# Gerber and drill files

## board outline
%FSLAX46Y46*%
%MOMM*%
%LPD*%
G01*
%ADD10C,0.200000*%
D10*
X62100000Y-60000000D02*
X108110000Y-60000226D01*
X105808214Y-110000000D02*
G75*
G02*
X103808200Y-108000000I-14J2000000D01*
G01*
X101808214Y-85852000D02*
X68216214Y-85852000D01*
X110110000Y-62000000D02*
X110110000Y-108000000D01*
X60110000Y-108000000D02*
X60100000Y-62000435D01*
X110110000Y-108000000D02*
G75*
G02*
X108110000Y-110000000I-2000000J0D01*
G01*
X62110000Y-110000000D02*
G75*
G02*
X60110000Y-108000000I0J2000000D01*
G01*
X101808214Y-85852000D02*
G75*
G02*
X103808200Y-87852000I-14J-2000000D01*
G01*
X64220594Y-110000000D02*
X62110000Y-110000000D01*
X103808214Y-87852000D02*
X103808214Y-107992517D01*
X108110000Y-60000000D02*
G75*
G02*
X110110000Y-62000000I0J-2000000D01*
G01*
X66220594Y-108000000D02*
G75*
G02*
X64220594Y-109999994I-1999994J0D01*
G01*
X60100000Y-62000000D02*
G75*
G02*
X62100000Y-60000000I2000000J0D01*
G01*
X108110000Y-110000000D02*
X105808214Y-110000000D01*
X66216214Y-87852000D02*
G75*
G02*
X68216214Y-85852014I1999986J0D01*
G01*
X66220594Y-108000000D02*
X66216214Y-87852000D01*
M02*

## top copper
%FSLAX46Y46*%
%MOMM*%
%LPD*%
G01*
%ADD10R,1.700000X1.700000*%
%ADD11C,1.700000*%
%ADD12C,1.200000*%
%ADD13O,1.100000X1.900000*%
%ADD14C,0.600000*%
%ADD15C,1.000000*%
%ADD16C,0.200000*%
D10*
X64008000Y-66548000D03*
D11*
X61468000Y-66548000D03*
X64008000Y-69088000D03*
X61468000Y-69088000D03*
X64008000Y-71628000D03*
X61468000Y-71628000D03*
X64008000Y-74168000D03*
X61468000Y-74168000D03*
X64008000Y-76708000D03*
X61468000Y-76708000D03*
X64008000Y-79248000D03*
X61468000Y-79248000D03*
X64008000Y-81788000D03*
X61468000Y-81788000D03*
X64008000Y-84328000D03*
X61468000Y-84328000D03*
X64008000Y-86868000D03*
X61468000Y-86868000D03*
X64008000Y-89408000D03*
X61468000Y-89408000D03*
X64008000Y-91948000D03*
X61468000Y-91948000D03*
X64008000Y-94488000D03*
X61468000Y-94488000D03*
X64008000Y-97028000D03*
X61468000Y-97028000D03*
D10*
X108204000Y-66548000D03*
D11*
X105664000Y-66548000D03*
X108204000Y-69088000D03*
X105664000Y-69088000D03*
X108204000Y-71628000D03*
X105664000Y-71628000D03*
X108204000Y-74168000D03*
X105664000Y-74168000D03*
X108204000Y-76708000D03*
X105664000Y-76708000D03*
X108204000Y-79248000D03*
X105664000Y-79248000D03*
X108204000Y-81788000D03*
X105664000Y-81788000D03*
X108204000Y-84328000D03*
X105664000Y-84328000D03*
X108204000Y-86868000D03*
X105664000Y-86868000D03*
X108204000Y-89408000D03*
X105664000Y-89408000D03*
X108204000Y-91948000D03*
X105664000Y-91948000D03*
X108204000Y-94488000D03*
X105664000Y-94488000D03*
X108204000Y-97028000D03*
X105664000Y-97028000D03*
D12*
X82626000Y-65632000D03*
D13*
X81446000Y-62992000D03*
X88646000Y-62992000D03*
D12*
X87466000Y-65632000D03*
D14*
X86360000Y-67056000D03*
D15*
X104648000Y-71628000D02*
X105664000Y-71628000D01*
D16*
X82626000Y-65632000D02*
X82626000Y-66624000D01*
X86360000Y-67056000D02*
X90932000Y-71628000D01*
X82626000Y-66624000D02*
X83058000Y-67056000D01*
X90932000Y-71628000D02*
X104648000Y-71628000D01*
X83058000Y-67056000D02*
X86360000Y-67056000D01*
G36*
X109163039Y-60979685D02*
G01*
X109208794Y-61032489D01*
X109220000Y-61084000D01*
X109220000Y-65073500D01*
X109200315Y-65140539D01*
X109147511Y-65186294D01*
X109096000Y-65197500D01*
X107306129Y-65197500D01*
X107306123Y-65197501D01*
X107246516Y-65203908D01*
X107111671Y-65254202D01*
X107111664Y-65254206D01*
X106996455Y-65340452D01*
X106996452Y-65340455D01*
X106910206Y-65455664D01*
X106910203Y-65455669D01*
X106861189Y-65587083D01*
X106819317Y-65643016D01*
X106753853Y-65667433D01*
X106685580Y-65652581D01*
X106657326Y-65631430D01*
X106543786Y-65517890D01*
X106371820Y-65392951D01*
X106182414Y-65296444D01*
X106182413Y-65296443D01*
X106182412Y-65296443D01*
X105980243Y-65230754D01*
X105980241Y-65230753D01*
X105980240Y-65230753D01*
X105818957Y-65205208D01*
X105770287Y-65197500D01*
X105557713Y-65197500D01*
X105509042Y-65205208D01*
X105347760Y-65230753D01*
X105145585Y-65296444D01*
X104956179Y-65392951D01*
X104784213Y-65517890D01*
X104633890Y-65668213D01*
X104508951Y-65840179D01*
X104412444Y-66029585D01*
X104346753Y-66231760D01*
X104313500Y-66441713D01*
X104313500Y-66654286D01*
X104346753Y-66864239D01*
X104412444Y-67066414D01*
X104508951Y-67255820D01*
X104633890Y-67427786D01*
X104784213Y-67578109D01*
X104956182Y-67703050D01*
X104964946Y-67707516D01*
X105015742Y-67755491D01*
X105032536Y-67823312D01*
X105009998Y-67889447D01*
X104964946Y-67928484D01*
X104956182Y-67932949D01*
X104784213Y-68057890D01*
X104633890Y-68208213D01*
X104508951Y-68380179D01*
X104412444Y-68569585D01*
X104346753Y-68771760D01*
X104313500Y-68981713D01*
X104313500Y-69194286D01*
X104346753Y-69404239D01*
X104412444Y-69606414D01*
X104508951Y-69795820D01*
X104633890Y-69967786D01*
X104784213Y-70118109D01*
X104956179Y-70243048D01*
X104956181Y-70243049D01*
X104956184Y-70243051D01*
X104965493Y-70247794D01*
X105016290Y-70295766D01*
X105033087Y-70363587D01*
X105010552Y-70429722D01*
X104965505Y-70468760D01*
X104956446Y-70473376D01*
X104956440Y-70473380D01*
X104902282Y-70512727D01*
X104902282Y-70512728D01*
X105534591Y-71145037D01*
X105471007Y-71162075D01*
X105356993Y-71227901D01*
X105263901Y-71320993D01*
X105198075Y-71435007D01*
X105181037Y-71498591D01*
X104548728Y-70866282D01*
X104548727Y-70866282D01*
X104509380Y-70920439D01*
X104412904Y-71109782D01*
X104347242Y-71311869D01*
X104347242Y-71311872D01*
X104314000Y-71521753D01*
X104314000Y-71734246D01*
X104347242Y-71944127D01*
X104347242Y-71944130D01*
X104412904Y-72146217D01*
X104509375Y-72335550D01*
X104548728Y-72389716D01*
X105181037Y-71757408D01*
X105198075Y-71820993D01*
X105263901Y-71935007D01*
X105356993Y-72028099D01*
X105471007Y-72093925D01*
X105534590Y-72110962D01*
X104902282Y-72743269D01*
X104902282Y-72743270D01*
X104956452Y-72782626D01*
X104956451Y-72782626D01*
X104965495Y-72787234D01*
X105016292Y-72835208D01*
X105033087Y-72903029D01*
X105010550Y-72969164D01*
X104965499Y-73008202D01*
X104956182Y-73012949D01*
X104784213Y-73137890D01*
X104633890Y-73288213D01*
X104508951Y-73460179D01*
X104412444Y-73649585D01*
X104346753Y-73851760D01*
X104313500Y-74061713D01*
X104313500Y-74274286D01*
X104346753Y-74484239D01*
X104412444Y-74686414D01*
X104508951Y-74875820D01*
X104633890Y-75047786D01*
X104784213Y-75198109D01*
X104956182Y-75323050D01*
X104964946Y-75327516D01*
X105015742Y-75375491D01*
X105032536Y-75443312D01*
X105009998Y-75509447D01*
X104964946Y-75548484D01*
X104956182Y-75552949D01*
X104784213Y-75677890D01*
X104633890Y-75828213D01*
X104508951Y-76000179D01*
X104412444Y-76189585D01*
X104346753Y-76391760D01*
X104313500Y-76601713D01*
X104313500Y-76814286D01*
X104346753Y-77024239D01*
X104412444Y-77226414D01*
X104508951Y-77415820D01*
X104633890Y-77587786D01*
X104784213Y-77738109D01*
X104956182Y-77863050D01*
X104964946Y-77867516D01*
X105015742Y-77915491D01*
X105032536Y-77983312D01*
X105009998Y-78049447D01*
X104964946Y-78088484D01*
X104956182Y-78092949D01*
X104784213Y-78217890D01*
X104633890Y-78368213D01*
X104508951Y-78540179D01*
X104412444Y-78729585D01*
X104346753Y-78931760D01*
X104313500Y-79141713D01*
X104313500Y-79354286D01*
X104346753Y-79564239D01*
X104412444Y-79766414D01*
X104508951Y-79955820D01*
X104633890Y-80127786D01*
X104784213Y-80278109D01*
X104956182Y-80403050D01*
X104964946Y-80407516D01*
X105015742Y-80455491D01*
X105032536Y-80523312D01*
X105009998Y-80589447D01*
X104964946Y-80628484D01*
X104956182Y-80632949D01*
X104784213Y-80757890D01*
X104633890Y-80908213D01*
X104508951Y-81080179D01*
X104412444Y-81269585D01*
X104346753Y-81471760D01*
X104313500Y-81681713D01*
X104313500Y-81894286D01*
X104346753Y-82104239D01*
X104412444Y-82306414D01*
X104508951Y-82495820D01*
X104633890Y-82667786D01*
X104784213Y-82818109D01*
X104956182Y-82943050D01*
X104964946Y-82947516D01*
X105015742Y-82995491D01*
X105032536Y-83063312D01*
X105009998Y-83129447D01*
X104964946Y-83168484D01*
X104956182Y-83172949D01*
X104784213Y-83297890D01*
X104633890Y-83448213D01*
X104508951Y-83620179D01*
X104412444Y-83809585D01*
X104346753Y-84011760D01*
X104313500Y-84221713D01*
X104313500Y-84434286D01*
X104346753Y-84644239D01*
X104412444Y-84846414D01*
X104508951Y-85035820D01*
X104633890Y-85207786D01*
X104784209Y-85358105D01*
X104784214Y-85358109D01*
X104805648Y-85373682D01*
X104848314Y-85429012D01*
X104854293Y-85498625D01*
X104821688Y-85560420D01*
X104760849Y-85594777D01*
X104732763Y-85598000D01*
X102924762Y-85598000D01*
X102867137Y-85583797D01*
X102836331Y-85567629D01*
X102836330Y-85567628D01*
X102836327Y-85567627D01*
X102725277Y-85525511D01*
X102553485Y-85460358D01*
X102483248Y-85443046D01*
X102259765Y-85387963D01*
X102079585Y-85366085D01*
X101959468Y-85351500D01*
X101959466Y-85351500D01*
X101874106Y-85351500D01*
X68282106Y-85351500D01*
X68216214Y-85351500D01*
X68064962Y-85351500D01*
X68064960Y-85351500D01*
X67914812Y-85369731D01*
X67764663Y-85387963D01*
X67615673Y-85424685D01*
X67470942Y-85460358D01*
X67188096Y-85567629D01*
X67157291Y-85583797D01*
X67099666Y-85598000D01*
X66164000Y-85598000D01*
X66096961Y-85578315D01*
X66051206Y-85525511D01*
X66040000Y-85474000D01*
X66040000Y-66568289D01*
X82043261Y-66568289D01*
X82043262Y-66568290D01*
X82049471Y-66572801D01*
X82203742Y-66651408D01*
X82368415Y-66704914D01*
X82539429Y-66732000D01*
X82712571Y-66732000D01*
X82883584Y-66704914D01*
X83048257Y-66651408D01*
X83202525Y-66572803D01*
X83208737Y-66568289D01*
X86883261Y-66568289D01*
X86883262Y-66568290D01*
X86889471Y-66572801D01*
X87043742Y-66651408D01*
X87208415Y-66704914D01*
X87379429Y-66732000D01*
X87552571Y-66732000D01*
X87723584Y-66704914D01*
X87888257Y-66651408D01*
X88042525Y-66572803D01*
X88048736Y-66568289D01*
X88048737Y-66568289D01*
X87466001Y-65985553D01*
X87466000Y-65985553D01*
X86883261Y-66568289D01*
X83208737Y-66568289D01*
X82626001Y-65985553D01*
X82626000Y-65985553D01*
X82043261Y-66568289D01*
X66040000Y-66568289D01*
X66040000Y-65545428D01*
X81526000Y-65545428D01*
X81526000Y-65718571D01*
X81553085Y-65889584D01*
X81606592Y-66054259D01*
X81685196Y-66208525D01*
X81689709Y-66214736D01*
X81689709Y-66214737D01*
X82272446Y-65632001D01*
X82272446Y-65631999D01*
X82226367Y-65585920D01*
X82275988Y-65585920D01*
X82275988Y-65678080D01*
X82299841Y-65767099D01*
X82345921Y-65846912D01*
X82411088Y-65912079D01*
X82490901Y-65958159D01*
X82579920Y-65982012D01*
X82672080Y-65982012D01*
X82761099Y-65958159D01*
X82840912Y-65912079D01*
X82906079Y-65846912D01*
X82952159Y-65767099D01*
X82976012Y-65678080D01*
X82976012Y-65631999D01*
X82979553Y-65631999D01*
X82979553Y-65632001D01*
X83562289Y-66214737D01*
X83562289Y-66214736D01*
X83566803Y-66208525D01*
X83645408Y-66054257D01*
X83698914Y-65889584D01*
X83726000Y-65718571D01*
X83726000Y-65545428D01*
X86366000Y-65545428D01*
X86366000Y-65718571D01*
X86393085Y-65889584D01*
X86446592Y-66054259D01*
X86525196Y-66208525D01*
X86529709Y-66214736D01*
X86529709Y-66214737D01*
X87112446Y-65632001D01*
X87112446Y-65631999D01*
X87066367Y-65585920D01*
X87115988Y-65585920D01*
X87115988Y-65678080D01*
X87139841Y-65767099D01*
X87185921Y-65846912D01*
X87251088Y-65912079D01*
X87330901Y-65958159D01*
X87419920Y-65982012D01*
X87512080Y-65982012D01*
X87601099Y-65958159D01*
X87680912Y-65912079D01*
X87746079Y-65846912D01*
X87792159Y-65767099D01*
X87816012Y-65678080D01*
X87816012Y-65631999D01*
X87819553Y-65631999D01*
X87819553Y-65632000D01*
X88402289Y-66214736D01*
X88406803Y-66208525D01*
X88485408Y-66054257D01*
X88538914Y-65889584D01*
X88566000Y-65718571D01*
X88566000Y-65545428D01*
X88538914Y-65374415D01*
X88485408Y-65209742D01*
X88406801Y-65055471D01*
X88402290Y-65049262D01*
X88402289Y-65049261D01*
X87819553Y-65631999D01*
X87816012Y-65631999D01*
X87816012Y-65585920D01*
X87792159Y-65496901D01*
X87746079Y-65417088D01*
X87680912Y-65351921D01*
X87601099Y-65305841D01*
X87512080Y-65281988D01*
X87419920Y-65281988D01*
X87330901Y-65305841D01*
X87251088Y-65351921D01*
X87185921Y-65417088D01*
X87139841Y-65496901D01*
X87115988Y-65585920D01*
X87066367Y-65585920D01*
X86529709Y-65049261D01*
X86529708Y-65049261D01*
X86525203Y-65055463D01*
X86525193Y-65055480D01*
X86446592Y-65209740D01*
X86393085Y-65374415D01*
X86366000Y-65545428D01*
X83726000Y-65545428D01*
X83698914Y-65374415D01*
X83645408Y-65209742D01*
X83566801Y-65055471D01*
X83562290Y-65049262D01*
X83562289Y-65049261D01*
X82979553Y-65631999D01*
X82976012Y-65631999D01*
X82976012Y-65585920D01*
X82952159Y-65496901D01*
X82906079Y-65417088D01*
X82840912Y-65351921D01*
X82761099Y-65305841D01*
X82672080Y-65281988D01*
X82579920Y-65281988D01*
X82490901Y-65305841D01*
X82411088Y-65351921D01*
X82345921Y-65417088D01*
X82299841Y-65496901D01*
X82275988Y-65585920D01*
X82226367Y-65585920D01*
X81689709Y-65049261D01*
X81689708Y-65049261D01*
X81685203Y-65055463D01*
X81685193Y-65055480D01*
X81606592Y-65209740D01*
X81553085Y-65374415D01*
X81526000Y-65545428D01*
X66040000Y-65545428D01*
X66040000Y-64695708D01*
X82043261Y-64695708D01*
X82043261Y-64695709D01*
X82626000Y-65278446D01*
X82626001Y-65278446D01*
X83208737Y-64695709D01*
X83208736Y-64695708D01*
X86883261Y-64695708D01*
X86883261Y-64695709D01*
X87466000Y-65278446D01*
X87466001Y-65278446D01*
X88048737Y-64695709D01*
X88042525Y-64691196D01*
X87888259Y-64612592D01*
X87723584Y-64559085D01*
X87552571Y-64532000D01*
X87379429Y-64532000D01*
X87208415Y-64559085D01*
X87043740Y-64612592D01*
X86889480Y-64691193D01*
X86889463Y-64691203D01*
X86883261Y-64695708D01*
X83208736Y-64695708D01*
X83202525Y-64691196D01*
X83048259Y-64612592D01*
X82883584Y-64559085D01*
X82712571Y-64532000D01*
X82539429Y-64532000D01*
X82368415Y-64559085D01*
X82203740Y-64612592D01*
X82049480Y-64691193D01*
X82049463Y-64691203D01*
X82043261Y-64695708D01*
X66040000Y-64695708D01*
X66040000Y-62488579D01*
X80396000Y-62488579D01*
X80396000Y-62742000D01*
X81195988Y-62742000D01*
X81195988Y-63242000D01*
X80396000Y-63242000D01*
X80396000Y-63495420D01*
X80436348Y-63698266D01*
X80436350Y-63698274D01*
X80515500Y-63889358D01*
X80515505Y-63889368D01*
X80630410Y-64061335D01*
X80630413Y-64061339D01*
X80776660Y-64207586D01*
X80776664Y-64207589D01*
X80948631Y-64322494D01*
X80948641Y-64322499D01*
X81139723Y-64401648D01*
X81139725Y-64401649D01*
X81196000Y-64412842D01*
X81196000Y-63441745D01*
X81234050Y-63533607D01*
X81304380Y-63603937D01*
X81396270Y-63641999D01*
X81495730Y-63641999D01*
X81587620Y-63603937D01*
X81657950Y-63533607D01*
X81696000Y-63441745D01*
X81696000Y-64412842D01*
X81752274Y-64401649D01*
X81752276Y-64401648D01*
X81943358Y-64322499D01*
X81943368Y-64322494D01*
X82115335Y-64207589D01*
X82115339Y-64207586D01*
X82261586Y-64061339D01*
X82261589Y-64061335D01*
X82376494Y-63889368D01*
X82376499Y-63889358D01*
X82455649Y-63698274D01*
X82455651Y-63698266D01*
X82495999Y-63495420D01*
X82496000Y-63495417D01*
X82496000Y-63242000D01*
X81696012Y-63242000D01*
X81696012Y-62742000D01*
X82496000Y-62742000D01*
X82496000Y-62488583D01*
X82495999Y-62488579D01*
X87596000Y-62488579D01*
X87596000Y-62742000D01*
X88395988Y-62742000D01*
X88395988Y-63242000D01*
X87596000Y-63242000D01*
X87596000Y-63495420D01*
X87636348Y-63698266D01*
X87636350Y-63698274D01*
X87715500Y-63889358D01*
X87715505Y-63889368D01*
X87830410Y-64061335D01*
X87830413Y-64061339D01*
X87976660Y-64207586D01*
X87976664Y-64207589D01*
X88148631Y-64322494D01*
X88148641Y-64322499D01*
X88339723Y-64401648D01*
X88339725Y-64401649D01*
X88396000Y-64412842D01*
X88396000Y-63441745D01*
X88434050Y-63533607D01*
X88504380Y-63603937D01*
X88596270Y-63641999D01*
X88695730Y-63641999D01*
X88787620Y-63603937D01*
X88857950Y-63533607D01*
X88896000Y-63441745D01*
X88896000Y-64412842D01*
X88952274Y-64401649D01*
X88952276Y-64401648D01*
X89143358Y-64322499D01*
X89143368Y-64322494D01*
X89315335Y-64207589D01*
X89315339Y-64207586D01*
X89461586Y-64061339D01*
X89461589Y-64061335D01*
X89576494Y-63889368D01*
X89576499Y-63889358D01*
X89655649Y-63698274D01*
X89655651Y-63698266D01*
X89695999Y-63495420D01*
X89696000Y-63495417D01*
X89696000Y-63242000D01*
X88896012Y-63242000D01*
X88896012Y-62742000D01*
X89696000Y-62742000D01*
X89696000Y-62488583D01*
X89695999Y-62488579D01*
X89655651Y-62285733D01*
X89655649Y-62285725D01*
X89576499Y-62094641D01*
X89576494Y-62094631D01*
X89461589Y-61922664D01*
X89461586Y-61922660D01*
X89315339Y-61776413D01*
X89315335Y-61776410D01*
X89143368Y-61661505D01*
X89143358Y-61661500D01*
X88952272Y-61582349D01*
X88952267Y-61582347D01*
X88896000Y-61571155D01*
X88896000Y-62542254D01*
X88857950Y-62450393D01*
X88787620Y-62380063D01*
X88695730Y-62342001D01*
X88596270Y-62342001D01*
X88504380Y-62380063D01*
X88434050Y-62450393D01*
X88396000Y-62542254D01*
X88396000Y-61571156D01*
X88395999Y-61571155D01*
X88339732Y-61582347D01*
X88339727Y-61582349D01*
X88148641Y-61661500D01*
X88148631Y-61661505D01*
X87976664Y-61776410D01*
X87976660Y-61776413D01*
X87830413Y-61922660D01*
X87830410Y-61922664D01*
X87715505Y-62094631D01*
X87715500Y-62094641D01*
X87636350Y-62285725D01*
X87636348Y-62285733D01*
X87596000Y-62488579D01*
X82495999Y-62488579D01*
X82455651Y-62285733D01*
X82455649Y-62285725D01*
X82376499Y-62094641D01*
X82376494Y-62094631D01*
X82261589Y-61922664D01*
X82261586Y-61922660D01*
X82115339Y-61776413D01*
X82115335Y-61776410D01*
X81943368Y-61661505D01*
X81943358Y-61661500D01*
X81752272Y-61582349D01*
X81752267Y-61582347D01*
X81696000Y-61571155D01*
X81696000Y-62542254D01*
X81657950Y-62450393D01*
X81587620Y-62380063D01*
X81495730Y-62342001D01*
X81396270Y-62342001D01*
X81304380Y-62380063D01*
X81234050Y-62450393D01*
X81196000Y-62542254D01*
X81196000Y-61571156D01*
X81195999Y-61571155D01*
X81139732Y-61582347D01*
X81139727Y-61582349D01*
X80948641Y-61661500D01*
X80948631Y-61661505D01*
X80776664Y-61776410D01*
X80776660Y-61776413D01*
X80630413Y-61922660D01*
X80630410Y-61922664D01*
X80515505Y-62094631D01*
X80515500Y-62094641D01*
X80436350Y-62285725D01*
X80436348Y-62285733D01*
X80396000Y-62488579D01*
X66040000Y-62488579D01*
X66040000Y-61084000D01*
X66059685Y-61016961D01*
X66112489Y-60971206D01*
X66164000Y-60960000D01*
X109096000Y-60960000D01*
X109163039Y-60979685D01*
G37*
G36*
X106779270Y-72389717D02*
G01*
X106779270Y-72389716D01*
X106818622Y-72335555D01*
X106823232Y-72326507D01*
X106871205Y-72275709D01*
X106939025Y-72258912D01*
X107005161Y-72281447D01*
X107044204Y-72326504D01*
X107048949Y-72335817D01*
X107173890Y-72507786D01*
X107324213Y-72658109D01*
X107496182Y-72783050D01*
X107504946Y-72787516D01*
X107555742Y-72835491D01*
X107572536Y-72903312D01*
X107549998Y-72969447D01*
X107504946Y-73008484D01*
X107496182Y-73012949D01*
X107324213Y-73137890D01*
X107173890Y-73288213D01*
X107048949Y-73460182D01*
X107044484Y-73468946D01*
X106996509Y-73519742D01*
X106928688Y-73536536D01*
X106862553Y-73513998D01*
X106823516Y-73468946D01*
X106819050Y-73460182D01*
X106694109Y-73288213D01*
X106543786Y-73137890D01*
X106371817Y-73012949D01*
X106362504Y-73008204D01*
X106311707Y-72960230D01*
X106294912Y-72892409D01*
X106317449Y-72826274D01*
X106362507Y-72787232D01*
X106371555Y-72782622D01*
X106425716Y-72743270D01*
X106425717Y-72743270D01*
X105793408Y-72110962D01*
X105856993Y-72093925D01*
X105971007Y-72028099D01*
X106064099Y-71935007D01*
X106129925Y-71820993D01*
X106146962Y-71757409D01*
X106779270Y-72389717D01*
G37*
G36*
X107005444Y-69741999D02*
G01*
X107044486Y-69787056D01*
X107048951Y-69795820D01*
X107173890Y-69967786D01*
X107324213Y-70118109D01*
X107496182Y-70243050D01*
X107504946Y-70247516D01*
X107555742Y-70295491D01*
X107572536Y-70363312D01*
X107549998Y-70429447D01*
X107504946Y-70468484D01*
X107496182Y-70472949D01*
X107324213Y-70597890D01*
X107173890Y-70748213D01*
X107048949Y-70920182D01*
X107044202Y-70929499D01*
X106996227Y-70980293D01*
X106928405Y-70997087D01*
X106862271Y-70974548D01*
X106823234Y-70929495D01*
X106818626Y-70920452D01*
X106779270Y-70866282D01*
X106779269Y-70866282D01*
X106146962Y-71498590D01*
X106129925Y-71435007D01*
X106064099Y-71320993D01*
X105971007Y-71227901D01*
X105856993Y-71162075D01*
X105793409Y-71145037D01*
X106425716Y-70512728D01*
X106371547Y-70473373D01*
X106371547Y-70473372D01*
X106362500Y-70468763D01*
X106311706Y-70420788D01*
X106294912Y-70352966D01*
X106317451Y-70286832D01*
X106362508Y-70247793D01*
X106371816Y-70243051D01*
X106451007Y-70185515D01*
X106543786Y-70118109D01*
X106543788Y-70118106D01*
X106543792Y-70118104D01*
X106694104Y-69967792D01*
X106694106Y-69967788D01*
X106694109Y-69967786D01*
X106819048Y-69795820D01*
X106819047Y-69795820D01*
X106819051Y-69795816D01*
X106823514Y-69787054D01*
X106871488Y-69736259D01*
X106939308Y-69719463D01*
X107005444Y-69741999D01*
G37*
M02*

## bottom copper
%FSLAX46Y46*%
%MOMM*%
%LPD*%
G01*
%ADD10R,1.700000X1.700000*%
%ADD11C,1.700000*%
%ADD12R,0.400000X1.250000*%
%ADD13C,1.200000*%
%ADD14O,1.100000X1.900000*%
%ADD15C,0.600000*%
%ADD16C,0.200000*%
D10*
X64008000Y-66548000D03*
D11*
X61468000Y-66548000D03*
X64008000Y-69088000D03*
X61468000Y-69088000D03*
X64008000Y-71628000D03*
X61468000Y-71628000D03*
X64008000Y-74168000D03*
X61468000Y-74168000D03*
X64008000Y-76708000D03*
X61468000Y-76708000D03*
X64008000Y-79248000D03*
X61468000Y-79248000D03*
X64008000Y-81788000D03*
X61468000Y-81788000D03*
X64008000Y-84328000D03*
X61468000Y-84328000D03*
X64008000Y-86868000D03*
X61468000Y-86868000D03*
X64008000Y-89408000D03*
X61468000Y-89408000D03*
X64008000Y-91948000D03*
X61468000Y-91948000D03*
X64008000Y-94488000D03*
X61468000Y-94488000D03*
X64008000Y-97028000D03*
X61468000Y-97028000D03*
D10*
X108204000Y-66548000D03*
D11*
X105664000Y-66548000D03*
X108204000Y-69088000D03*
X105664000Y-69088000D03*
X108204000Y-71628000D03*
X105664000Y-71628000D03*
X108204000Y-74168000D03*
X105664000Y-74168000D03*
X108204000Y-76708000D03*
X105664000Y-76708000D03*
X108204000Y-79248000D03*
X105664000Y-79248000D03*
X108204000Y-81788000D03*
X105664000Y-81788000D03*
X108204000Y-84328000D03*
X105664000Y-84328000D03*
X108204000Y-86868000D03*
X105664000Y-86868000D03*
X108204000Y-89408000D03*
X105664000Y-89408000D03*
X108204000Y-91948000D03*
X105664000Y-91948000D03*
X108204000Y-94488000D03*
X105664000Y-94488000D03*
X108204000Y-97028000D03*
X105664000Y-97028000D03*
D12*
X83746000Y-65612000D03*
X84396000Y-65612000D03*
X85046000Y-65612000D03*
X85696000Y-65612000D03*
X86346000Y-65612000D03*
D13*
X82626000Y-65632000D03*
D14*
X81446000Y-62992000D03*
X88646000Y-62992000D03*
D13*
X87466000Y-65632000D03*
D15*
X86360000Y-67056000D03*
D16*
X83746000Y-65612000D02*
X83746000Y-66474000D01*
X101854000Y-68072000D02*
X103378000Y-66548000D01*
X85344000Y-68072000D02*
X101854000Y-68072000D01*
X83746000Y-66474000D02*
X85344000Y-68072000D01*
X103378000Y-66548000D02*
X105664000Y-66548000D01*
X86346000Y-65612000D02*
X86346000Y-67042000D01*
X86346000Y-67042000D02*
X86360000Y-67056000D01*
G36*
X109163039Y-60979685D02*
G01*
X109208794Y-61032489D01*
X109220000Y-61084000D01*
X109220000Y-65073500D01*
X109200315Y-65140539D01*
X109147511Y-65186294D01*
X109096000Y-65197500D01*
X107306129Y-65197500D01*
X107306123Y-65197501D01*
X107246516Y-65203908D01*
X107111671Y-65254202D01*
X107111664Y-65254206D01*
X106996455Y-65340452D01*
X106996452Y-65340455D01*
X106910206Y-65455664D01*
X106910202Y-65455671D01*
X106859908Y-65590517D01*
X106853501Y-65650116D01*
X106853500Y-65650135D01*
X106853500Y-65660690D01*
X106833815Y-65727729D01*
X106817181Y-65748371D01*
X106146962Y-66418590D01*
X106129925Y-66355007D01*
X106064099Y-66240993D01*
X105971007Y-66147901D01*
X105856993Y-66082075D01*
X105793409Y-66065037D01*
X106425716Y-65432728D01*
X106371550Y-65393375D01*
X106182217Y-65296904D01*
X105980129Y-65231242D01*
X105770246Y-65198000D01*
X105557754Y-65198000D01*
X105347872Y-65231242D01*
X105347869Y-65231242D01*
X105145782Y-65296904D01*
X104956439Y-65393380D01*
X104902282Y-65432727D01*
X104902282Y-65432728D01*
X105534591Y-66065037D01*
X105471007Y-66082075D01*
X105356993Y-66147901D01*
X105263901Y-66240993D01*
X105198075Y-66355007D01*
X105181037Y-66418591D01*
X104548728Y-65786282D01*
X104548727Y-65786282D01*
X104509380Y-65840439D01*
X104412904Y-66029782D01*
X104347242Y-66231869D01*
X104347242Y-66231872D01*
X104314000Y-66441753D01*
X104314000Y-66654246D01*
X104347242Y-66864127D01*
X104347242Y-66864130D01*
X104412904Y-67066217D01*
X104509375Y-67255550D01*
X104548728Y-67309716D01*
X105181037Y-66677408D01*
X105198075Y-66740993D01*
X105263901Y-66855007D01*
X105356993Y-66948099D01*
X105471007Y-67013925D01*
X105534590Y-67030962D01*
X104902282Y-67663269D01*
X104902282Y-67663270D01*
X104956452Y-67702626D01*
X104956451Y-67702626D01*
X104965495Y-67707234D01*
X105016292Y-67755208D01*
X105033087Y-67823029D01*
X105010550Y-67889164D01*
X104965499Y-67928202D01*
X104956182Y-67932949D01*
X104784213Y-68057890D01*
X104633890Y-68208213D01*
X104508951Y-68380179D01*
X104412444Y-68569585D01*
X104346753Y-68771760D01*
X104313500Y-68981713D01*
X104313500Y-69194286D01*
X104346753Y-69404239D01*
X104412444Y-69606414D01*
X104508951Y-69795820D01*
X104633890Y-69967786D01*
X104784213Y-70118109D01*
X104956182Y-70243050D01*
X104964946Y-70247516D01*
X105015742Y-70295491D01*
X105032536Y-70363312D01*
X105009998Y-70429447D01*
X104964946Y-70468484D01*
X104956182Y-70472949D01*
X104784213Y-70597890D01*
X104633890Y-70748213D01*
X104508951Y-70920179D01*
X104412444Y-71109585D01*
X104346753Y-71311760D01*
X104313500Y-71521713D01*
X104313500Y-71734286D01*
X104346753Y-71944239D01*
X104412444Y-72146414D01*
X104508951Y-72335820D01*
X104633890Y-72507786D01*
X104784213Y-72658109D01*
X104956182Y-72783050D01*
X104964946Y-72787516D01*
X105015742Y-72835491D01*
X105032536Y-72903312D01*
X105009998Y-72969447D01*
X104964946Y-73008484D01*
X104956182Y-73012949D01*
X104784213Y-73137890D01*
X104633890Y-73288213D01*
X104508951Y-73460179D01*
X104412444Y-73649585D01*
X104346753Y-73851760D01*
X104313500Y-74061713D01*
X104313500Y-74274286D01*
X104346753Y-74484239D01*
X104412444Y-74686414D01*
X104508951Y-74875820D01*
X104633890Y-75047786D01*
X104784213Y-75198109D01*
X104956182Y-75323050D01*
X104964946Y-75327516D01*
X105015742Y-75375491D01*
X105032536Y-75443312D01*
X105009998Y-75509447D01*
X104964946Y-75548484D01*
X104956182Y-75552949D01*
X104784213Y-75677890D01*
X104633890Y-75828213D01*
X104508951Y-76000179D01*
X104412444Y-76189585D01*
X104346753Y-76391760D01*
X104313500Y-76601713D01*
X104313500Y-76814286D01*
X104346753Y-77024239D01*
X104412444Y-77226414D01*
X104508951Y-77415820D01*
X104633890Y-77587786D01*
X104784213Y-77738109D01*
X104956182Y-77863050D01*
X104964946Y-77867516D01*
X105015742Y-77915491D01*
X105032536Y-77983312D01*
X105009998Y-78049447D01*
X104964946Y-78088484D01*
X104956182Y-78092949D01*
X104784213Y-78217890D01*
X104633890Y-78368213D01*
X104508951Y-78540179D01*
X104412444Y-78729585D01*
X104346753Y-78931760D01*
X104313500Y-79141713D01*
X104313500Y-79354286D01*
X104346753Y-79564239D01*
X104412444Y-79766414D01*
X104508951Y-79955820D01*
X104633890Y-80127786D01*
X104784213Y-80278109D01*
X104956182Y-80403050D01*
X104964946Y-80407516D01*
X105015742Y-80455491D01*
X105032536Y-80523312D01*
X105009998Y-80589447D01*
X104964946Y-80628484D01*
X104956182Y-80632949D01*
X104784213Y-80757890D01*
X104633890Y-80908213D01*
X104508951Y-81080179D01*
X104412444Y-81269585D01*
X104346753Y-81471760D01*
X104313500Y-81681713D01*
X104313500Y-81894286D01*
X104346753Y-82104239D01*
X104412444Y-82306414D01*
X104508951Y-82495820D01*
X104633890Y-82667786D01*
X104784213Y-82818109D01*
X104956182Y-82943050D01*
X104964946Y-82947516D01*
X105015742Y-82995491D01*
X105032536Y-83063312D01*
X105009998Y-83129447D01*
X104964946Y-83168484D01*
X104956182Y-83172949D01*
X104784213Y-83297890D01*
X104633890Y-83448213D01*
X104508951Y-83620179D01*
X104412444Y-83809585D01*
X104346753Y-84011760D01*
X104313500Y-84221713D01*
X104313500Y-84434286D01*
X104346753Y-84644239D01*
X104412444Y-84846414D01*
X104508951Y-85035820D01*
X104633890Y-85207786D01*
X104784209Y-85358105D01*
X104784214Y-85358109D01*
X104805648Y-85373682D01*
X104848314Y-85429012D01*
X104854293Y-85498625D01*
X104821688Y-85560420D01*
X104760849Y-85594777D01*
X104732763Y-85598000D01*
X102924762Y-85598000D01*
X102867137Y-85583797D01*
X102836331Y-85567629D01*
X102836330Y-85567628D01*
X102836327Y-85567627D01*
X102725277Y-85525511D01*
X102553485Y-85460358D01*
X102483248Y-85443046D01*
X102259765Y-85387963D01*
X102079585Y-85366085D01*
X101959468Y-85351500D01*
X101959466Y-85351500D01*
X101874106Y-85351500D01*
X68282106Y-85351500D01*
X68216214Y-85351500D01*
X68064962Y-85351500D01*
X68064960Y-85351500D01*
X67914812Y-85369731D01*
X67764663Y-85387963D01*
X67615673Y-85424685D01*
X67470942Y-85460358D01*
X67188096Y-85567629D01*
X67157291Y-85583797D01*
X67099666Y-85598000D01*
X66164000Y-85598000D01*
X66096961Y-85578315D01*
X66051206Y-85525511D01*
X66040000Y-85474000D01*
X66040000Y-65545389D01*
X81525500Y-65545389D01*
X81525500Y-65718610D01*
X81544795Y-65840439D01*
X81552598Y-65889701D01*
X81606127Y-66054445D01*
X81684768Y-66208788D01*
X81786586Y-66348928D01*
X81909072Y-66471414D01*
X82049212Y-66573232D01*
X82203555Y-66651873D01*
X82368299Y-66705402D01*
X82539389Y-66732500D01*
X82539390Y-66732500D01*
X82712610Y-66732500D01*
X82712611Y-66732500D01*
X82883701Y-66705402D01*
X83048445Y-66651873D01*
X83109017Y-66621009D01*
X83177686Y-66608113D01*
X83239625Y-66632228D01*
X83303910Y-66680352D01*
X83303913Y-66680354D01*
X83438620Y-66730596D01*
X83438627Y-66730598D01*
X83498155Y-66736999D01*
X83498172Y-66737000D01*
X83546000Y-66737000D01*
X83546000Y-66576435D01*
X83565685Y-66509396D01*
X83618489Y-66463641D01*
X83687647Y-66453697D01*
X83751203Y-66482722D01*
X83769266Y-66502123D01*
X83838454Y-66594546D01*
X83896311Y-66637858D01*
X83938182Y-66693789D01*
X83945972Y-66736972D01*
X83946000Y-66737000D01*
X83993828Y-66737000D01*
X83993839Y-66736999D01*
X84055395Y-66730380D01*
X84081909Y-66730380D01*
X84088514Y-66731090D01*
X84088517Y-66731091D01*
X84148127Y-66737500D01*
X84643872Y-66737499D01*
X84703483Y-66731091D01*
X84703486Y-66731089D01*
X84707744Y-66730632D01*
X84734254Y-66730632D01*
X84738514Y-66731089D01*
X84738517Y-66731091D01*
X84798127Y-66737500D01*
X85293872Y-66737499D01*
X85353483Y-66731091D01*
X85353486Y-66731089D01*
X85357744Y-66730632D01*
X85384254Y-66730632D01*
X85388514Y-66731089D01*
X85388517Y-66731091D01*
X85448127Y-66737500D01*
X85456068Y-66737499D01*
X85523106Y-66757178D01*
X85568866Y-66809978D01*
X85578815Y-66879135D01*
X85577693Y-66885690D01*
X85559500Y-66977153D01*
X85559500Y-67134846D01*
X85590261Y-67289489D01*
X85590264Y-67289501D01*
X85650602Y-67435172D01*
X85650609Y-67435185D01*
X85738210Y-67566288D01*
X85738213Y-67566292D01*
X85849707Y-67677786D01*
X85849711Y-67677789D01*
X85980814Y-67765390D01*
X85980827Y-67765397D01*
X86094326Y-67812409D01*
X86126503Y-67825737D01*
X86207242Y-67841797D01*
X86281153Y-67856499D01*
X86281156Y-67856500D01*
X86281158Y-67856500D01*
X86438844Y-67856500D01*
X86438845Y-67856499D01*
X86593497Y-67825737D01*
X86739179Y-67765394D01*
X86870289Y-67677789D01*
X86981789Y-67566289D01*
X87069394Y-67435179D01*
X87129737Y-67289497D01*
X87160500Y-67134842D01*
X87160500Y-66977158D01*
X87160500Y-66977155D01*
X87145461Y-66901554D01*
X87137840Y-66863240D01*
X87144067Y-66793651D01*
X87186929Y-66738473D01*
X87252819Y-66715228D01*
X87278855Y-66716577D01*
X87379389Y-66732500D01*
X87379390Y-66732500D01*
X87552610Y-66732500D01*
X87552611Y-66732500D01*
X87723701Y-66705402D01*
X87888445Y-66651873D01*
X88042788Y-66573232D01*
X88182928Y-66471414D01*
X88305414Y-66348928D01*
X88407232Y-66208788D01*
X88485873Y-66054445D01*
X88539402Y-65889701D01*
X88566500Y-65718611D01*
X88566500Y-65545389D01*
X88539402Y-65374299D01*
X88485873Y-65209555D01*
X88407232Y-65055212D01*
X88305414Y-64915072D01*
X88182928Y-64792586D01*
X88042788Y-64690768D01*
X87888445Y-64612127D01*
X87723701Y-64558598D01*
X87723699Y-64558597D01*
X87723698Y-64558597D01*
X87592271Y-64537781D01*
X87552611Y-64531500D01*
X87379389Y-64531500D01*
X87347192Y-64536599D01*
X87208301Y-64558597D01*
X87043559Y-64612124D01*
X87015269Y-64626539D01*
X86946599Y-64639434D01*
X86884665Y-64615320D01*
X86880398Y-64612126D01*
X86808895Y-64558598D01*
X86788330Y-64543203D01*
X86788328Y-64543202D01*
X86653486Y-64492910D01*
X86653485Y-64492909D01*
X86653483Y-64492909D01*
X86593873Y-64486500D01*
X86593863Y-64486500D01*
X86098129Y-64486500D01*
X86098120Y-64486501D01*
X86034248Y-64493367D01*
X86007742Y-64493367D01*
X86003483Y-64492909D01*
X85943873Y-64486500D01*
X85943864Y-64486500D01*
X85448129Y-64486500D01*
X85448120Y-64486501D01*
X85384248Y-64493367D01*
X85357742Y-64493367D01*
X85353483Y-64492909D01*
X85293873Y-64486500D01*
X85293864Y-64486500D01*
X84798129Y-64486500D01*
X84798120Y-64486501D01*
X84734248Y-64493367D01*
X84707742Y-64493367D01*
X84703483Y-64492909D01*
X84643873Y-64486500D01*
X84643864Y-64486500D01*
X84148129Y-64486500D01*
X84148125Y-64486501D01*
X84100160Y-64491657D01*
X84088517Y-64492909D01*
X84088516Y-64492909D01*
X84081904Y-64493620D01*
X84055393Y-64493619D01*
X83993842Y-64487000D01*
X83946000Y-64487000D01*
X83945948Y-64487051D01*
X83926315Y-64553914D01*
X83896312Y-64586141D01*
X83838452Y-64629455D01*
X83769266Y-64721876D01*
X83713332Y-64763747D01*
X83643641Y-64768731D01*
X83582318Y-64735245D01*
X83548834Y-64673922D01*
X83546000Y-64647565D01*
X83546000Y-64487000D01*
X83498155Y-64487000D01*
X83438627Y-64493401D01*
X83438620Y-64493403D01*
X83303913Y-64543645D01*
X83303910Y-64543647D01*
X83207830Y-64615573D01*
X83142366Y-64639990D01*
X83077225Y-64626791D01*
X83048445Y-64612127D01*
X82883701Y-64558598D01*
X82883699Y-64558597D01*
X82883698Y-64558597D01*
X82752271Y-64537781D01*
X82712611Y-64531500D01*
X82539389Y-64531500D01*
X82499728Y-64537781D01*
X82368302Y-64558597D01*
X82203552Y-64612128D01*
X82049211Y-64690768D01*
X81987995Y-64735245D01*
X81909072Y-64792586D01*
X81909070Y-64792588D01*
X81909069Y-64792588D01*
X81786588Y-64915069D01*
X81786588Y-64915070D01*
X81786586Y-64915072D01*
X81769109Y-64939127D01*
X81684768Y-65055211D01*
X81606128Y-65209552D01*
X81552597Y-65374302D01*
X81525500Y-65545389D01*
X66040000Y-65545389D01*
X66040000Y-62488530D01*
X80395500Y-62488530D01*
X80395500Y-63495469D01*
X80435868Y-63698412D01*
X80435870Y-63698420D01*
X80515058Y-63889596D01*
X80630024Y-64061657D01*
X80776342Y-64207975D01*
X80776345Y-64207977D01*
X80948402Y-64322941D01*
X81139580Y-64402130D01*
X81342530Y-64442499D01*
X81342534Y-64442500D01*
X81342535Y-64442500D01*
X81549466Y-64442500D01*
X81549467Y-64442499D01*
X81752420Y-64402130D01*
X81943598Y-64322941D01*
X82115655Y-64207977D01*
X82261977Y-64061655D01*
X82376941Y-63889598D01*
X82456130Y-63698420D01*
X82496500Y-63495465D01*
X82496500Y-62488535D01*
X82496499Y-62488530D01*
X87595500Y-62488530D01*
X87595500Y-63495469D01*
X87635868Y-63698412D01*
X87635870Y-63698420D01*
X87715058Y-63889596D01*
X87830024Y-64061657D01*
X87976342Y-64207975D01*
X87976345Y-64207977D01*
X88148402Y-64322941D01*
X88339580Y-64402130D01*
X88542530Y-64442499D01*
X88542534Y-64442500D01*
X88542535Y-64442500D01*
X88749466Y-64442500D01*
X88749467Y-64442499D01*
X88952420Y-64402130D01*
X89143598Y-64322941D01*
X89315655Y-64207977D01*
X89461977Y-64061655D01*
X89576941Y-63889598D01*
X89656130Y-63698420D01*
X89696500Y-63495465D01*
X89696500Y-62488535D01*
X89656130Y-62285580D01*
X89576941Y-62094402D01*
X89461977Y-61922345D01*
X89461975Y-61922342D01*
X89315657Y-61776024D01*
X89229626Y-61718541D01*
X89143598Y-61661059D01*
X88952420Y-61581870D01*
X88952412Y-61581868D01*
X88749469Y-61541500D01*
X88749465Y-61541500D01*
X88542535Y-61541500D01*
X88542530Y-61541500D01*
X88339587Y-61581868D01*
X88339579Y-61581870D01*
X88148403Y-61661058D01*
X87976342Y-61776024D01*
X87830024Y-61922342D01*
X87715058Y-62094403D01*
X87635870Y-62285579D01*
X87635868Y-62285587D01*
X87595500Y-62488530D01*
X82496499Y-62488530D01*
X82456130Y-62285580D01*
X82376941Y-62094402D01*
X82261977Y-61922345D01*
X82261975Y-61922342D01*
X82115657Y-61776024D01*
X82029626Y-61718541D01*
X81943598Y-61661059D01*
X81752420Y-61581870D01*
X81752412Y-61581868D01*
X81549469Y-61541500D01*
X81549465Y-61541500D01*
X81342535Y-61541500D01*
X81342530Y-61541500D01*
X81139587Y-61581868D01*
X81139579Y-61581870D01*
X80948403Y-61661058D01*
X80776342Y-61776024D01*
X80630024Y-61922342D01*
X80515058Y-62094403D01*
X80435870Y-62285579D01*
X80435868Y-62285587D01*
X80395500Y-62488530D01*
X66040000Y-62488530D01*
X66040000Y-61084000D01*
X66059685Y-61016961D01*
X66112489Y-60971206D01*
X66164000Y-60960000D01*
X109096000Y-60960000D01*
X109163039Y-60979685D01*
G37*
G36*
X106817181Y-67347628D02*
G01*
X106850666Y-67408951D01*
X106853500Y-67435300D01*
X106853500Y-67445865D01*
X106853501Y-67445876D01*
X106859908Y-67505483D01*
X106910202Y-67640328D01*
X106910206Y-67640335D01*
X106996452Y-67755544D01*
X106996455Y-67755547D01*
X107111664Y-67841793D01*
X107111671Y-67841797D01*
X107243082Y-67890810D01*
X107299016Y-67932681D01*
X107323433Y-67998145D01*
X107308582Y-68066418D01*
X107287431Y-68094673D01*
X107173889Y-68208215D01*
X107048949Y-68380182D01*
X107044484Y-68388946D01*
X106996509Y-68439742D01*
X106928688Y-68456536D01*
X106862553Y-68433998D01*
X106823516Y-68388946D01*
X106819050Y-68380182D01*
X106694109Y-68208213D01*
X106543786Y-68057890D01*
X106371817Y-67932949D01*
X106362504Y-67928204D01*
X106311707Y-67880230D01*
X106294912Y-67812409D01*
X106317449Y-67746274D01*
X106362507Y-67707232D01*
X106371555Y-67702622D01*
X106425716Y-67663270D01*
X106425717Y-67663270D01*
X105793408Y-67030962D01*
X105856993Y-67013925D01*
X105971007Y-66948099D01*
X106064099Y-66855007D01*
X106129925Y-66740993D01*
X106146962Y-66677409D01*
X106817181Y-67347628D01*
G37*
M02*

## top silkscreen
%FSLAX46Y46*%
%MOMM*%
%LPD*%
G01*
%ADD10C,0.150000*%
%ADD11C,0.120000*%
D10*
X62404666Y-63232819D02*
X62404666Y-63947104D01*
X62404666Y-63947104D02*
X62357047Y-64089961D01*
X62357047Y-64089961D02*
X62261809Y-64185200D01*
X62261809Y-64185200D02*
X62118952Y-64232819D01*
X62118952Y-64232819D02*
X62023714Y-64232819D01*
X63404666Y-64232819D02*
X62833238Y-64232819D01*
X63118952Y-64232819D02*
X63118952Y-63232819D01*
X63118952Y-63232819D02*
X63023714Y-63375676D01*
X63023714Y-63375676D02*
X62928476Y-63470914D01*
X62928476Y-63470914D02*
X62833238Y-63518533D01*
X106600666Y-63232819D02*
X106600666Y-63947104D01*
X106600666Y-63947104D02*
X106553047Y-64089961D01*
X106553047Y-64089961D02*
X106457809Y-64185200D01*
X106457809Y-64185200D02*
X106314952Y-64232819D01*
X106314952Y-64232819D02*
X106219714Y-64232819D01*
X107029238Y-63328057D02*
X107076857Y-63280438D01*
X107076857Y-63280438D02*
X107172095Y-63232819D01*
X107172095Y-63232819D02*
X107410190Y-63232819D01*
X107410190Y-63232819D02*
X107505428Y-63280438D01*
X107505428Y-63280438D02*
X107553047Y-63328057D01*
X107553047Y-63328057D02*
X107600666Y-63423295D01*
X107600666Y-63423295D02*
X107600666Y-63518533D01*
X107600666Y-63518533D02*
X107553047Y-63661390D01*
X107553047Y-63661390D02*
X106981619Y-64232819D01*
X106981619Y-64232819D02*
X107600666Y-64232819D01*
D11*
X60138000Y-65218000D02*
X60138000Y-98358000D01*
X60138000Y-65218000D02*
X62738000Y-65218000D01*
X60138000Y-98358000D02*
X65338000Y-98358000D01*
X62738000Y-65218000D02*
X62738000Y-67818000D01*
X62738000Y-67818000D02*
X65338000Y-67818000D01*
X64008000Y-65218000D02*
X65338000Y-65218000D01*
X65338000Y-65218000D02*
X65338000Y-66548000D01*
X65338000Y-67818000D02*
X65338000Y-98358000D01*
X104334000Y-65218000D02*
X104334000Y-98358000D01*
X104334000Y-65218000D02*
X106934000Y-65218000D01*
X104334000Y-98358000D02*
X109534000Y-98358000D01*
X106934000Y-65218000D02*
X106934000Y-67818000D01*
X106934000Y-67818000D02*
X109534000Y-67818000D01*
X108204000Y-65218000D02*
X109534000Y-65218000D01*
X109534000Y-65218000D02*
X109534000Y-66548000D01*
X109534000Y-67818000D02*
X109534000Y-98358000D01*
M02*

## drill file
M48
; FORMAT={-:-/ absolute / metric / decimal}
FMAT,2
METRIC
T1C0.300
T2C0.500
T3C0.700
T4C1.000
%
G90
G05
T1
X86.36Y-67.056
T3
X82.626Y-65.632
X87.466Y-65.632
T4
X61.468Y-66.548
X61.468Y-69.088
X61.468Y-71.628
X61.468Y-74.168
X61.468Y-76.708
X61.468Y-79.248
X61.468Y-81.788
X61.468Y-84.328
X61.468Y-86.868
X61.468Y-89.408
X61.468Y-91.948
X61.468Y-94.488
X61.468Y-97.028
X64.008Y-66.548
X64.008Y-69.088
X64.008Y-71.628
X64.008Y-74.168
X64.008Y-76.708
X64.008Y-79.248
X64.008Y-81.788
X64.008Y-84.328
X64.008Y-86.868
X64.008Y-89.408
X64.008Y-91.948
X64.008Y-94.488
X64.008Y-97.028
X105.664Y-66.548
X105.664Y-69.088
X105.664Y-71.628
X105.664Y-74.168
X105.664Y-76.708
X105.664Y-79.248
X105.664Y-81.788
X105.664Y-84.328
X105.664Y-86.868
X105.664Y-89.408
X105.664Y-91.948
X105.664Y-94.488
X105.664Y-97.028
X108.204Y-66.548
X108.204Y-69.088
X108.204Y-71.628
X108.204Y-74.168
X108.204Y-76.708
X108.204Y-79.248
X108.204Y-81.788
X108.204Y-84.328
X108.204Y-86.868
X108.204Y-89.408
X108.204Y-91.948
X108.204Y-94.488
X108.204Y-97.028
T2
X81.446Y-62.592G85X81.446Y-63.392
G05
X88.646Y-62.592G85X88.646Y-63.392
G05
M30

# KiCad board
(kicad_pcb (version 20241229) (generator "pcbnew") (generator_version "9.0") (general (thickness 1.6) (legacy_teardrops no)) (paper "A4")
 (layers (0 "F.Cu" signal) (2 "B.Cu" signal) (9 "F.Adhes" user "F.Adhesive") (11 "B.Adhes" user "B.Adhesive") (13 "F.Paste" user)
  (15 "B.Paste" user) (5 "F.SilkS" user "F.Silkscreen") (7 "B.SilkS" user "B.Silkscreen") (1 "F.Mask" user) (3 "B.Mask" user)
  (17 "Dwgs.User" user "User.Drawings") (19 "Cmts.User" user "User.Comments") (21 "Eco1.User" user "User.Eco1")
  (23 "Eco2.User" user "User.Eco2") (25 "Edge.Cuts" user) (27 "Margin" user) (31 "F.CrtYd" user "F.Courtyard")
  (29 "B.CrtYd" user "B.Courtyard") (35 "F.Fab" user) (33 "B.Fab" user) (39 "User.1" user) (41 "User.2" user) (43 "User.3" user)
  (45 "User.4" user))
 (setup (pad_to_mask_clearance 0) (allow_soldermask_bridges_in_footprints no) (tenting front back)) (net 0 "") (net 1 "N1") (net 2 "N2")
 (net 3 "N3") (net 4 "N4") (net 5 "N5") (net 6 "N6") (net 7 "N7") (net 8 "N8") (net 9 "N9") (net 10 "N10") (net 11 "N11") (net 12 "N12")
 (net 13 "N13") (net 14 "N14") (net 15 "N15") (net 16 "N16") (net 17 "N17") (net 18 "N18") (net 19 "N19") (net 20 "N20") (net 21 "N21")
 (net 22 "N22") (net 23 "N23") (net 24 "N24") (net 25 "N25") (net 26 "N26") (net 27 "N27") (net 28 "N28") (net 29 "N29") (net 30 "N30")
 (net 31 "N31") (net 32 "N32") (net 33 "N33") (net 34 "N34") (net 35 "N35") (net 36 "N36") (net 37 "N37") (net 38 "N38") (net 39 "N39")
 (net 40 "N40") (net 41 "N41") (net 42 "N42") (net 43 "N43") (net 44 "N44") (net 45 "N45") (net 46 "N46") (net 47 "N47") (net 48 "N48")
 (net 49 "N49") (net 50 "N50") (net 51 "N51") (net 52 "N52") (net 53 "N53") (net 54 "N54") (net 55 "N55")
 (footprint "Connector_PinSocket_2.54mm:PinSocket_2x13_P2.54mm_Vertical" (layer "F.Cu") (at 64.008 66.548)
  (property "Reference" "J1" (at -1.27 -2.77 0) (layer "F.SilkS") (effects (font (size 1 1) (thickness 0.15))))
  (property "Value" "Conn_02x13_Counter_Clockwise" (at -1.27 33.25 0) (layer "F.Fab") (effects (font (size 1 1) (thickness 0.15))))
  (fp_line (start -3.87 -1.33) (end -3.87 31.81) (stroke (width 0.12) (type solid)) (layer "F.SilkS"))
  (fp_line (start -3.87 -1.33) (end -1.27 -1.33) (stroke (width 0.12) (type solid)) (layer "F.SilkS"))
  (fp_line (start -3.87 31.81) (end 1.33 31.81) (stroke (width 0.12) (type solid)) (layer "F.SilkS"))
  (fp_line (start -1.27 -1.33) (end -1.27 1.27) (stroke (width 0.12) (type solid)) (layer "F.SilkS"))
  (fp_line (start -1.27 1.27) (end 1.33 1.27) (stroke (width 0.12) (type solid)) (layer "F.SilkS"))
  (fp_line (start 0 -1.33) (end 1.33 -1.33) (stroke (width 0.12) (type solid)) (layer "F.SilkS"))
  (fp_line (start 1.33 -1.33) (end 1.33 0) (stroke (width 0.12) (type solid)) (layer "F.SilkS"))
  (fp_line (start 1.33 1.27) (end 1.33 31.81) (stroke (width 0.12) (type solid)) (layer "F.SilkS"))
  (pad "1" thru_hole rect (at 0 0) (size 1.7 1.7) (drill 1) (layers "*.Cu" "*.Mask") (remove_unused_layers no) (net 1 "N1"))
  (pad "2" thru_hole circle (at -2.54 0) (size 1.7 1.7) (drill 1) (layers "*.Cu" "*.Mask") (remove_unused_layers no) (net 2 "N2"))
  (pad "3" thru_hole circle (at 0 2.54) (size 1.7 1.7) (drill 1) (layers "*.Cu" "*.Mask") (remove_unused_layers no) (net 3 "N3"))
  (pad "4" thru_hole circle (at -2.54 2.54) (size 1.7 1.7) (drill 1) (layers "*.Cu" "*.Mask") (remove_unused_layers no) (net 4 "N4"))
  (pad "5" thru_hole circle (at 0 5.08) (size 1.7 1.7) (drill 1) (layers "*.Cu" "*.Mask") (remove_unused_layers no) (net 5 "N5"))
  (pad "6" thru_hole circle (at -2.54 5.08) (size 1.7 1.7) (drill 1) (layers "*.Cu" "*.Mask") (remove_unused_layers no) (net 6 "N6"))
  (pad "7" thru_hole circle (at 0 7.62) (size 1.7 1.7) (drill 1) (layers "*.Cu" "*.Mask") (remove_unused_layers no) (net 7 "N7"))
  (pad "8" thru_hole circle (at -2.54 7.62) (size 1.7 1.7) (drill 1) (layers "*.Cu" "*.Mask") (remove_unused_layers no) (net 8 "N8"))
  (pad "9" thru_hole circle (at 0 10.16) (size 1.7 1.7) (drill 1) (layers "*.Cu" "*.Mask") (remove_unused_layers no) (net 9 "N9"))
  (pad "10" thru_hole circle (at -2.54 10.16) (size 1.7 1.7) (drill 1) (layers "*.Cu" "*.Mask") (remove_unused_layers no) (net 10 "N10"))
  (pad "11" thru_hole circle (at 0 12.7) (size 1.7 1.7) (drill 1) (layers "*.Cu" "*.Mask") (remove_unused_layers no) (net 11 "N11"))
  (pad "12" thru_hole circle (at -2.54 12.7) (size 1.7 1.7) (drill 1) (layers "*.Cu" "*.Mask") (remove_unused_layers no) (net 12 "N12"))
  (pad "13" thru_hole circle (at 0 15.24) (size 1.7 1.7) (drill 1) (layers "*.Cu" "*.Mask") (remove_unused_layers no) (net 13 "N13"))
  (pad "14" thru_hole circle (at -2.54 15.24) (size 1.7 1.7) (drill 1) (layers "*.Cu" "*.Mask") (remove_unused_layers no) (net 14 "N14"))
  (pad "15" thru_hole circle (at 0 17.78) (size 1.7 1.7) (drill 1) (layers "*.Cu" "*.Mask") (remove_unused_layers no) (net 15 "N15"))
  (pad "16" thru_hole circle (at -2.54 17.78) (size 1.7 1.7) (drill 1) (layers "*.Cu" "*.Mask") (remove_unused_layers no) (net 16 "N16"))
  (pad "17" thru_hole circle (at 0 20.32) (size 1.7 1.7) (drill 1) (layers "*.Cu" "*.Mask") (remove_unused_layers no) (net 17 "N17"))
  (pad "18" thru_hole circle (at -2.54 20.32) (size 1.7 1.7) (drill 1) (layers "*.Cu" "*.Mask") (remove_unused_layers no) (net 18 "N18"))
  (pad "19" thru_hole circle (at 0 22.86) (size 1.7 1.7) (drill 1) (layers "*.Cu" "*.Mask") (remove_unused_layers no) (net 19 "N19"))
  (pad "20" thru_hole circle (at -2.54 22.86) (size 1.7 1.7) (drill 1) (layers "*.Cu" "*.Mask") (remove_unused_layers no) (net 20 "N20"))
  (pad "21" thru_hole circle (at 0 25.4) (size 1.7 1.7) (drill 1) (layers "*.Cu" "*.Mask") (remove_unused_layers no) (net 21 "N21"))
  (pad "22" thru_hole circle (at -2.54 25.4) (size 1.7 1.7) (drill 1) (layers "*.Cu" "*.Mask") (remove_unused_layers no) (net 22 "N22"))
  (pad "23" thru_hole circle (at 0 27.94) (size 1.7 1.7) (drill 1) (layers "*.Cu" "*.Mask") (remove_unused_layers no) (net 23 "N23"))
  (pad "24" thru_hole circle (at -2.54 27.94) (size 1.7 1.7) (drill 1) (layers "*.Cu" "*.Mask") (remove_unused_layers no) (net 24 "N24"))
  (pad "25" thru_hole circle (at 0 30.48) (size 1.7 1.7) (drill 1) (layers "*.Cu" "*.Mask") (remove_unused_layers no) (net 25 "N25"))
  (pad "26" thru_hole circle (at -2.54 30.48) (size 1.7 1.7) (drill 1) (layers "*.Cu" "*.Mask") (remove_unused_layers no) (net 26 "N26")))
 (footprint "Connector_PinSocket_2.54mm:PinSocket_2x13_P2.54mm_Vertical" (layer "F.Cu") (at 108.204 66.548)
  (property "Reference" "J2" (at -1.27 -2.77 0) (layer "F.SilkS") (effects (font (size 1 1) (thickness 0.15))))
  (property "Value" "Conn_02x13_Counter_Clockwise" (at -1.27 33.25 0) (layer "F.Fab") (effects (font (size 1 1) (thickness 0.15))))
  (fp_line (start -3.87 -1.33) (end -3.87 31.81) (stroke (width 0.12) (type solid)) (layer "F.SilkS"))
  (fp_line (start -3.87 -1.33) (end -1.27 -1.33) (stroke (width 0.12) (type solid)) (layer "F.SilkS"))
  (fp_line (start -3.87 31.81) (end 1.33 31.81) (stroke (width 0.12) (type solid)) (layer "F.SilkS"))
  (fp_line (start -1.27 -1.33) (end -1.27 1.27) (stroke (width 0.12) (type solid)) (layer "F.SilkS"))
  (fp_line (start -1.27 1.27) (end 1.33 1.27) (stroke (width 0.12) (type solid)) (layer "F.SilkS"))
  (fp_line (start 0 -1.33) (end 1.33 -1.33) (stroke (width 0.12) (type solid)) (layer "F.SilkS"))
  (fp_line (start 1.33 -1.33) (end 1.33 0) (stroke (width 0.12) (type solid)) (layer "F.SilkS"))
  (fp_line (start 1.33 1.27) (end 1.33 31.81) (stroke (width 0.12) (type solid)) (layer "F.SilkS"))
  (pad "1" thru_hole rect (at 0 0) (size 1.7 1.7) (drill 1) (layers "*.Cu" "*.Mask") (remove_unused_layers no) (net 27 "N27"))
  (pad "2" thru_hole circle (at -2.54 0) (size 1.7 1.7) (drill 1) (layers "*.Cu" "*.Mask") (remove_unused_layers no) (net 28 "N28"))
  (pad "3" thru_hole circle (at 0 2.54) (size 1.7 1.7) (drill 1) (layers "*.Cu" "*.Mask") (remove_unused_layers no) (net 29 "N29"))
  (pad "4" thru_hole circle (at -2.54 2.54) (size 1.7 1.7) (drill 1) (layers "*.Cu" "*.Mask") (remove_unused_layers no) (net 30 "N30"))
  (pad "5" thru_hole circle (at 0 5.08) (size 1.7 1.7) (drill 1) (layers "*.Cu" "*.Mask") (remove_unused_layers no) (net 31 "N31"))
  (pad "6" thru_hole circle (at -2.54 5.08) (size 1.7 1.7) (drill 1) (layers "*.Cu" "*.Mask") (remove_unused_layers no) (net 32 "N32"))
  (pad "7" thru_hole circle (at 0 7.62) (size 1.7 1.7) (drill 1) (layers "*.Cu" "*.Mask") (remove_unused_layers no) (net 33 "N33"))
  (pad "8" thru_hole circle (at -2.54 7.62) (size 1.7 1.7) (drill 1) (layers "*.Cu" "*.Mask") (remove_unused_layers no) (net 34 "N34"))
  (pad "9" thru_hole circle (at 0 10.16) (size 1.7 1.7) (drill 1) (layers "*.Cu" "*.Mask") (remove_unused_layers no) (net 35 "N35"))
  (pad "10" thru_hole circle (at -2.54 10.16) (size 1.7 1.7) (drill 1) (layers "*.Cu" "*.Mask") (remove_unused_layers no) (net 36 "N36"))
  (pad "11" thru_hole circle (at 0 12.7) (size 1.7 1.7) (drill 1) (layers "*.Cu" "*.Mask") (remove_unused_layers no) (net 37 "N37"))
  (pad "12" thru_hole circle (at -2.54 12.7) (size 1.7 1.7) (drill 1) (layers "*.Cu" "*.Mask") (remove_unused_layers no) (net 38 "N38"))
  (pad "13" thru_hole circle (at 0 15.24) (size 1.7 1.7) (drill 1) (layers "*.Cu" "*.Mask") (remove_unused_layers no) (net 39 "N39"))
  (pad "14" thru_hole circle (at -2.54 15.24) (size 1.7 1.7) (drill 1) (layers "*.Cu" "*.Mask") (remove_unused_layers no) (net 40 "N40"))
  (pad "15" thru_hole circle (at 0 17.78) (size 1.7 1.7) (drill 1) (layers "*.Cu" "*.Mask") (remove_unused_layers no) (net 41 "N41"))
  (pad "16" thru_hole circle (at -2.54 17.78) (size 1.7 1.7) (drill 1) (layers "*.Cu" "*.Mask") (remove_unused_layers no) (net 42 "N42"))
  (pad "17" thru_hole circle (at 0 20.32) (size 1.7 1.7) (drill 1) (layers "*.Cu" "*.Mask") (remove_unused_layers no) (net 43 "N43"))
  (pad "18" thru_hole circle (at -2.54 20.32) (size 1.7 1.7) (drill 1) (layers "*.Cu" "*.Mask") (remove_unused_layers no) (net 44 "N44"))
  (pad "19" thru_hole circle (at 0 22.86) (size 1.7 1.7) (drill 1) (layers "*.Cu" "*.Mask") (remove_unused_layers no) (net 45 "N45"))
  (pad "20" thru_hole circle (at -2.54 22.86) (size 1.7 1.7) (drill 1) (layers "*.Cu" "*.Mask") (remove_unused_layers no) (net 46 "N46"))
  (pad "21" thru_hole circle (at 0 25.4) (size 1.7 1.7) (drill 1) (layers "*.Cu" "*.Mask") (remove_unused_layers no) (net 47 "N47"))
  (pad "22" thru_hole circle (at -2.54 25.4) (size 1.7 1.7) (drill 1) (layers "*.Cu" "*.Mask") (remove_unused_layers no) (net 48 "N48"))
  (pad "23" thru_hole circle (at 0 27.94) (size 1.7 1.7) (drill 1) (layers "*.Cu" "*.Mask") (remove_unused_layers no) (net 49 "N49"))
  (pad "24" thru_hole circle (at -2.54 27.94) (size 1.7 1.7) (drill 1) (layers "*.Cu" "*.Mask") (remove_unused_layers no) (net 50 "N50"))
  (pad "25" thru_hole circle (at 0 30.48) (size 1.7 1.7) (drill 1) (layers "*.Cu" "*.Mask") (remove_unused_layers no) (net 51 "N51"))
  (pad "26" thru_hole circle (at -2.54 30.48) (size 1.7 1.7) (drill 1) (layers "*.Cu" "*.Mask") (remove_unused_layers no) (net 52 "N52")))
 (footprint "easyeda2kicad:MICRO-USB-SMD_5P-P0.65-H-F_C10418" (layer "B.Cu") (at 85.046 64.312)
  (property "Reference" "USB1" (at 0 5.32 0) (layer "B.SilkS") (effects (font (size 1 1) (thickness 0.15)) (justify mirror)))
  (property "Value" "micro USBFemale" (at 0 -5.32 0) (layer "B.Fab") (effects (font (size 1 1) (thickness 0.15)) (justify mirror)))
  (pad "1" smd rect (at -1.3 1.3 90) (size 1.25 0.4) (layers "B.Cu" "B.Mask" "B.Paste") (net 28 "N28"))
  (pad "2" smd rect (at -0.65 1.3 90) (size 1.25 0.4) (layers "B.Cu" "B.Mask" "B.Paste") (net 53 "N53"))
  (pad "3" smd rect (at 0 1.3 90) (size 1.25 0.4) (layers "B.Cu" "B.Mask" "B.Paste") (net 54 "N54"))
  (pad "4" smd rect (at 0.65 1.3 90) (size 1.25 0.4) (layers "B.Cu" "B.Mask" "B.Paste") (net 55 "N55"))
  (pad "5" smd rect (at 1.3 1.3 90) (size 1.25 0.4) (layers "B.Cu" "B.Mask" "B.Paste") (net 32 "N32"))
  (pad "SH0" thru_hole circle (at -2.42 1.32) (size 1.2 1.2) (drill 0.700024) (layers "*.Cu" "*.Mask") (remove_unused_layers no)
   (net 32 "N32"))
  (pad "SH1" thru_hole oval (at -3.6 -1.32) (size 1.1 1.9) (drill oval 0.500024 1.299997) (layers "*.Cu" "*.Mask") (remove_unused_layers no)
   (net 32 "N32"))
  (pad "SH2" thru_hole oval (at 3.6 -1.32) (size 1.1 1.9) (drill oval 0.500024 1.299997) (layers "*.Cu" "*.Mask") (remove_unused_layers no)
   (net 32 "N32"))
  (pad "SH3" thru_hole circle (at 2.42 1.32) (size 1.2 1.2) (drill 0.700024) (layers "*.Cu" "*.Mask") (remove_unused_layers no)
   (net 32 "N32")))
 (gr_line (start 62.1 60) (end 108.11 60.000226) (stroke (width 0.2) (type solid)) (layer "Edge.Cuts"))
 (gr_arc (start 105.808214 110) (mid 104.394 109.414214) (end 103.808214 108) (stroke (width 0.2) (type solid)) (layer "Edge.Cuts"))
 (gr_line (start 101.808214 85.852) (end 68.216214 85.852) (stroke (width 0.2) (type solid)) (layer "Edge.Cuts"))
 (gr_line (start 110.11 62) (end 110.11 108) (stroke (width 0.2) (type solid)) (layer "Edge.Cuts"))
 (gr_line (start 60.11 108) (end 60.1 62.000435) (stroke (width 0.2) (type solid)) (layer "Edge.Cuts"))
 (gr_arc (start 110.11 108) (mid 109.524214 109.414214) (end 108.11 110) (stroke (width 0.2) (type solid)) (layer "Edge.Cuts"))
 (gr_arc (start 62.11 110) (mid 60.695786 109.414214) (end 60.11 108) (stroke (width 0.2) (type solid)) (layer "Edge.Cuts"))
 (gr_arc (start 101.808214 85.852) (mid 103.222428 86.437786) (end 103.808214 87.852) (stroke (width 0.2) (type solid)) (layer "Edge.Cuts"))
 (gr_line (start 64.220594 110) (end 62.11 110) (stroke (width 0.2) (type solid)) (layer "Edge.Cuts"))
 (gr_line (start 103.808214 87.852) (end 103.808214 107.992517) (stroke (width 0.2) (type solid)) (layer "Edge.Cuts"))
 (gr_arc (start 108.11 60) (mid 109.524214 60.585786) (end 110.11 62) (stroke (width 0.2) (type solid)) (layer "Edge.Cuts"))
 (gr_arc (start 66.220594 108) (mid 65.634808 109.414214) (end 64.220594 110) (stroke (width 0.2) (type solid)) (layer "Edge.Cuts"))
 (gr_arc (start 60.1 62) (mid 60.685786 60.585786) (end 62.1 60) (stroke (width 0.2) (type solid)) (layer "Edge.Cuts"))
 (gr_line (start 108.11 110) (end 105.808214 110) (stroke (width 0.2) (type solid)) (layer "Edge.Cuts"))
 (gr_arc (start 66.216214 87.852) (mid 66.802 86.437786) (end 68.216214 85.852) (stroke (width 0.2) (type solid)) (layer "Edge.Cuts"))
 (gr_line (start 66.220594 108) (end 66.216214 87.852) (stroke (width 0.2) (type solid)) (layer "Edge.Cuts"))
 (segment (start 83.746 65.612) (end 83.746 66.474) (width 0.2) (layer "B.Cu") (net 28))
 (segment (start 101.854 68.072) (end 103.378 66.548) (width 0.2) (layer "B.Cu") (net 28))
 (segment (start 85.344 68.072) (end 101.854 68.072) (width 0.2) (layer "B.Cu") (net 28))
 (segment (start 83.746 66.474) (end 85.344 68.072) (width 0.2) (layer "B.Cu") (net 28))
 (segment (start 103.378 66.548) (end 105.664 66.548) (width 0.2) (layer "B.Cu") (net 28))
 (segment (start 104.648 71.628) (end 105.664 71.628) (width 1) (layer "F.Cu") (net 32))
 (segment (start 82.626 65.632) (end 82.626 66.624) (width 0.2) (layer "F.Cu") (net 32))
 (segment (start 86.36 67.056) (end 90.932 71.628) (width 0.2) (layer "F.Cu") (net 32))
 (segment (start 82.626 66.624) (end 83.058 67.056) (width 0.2) (layer "F.Cu") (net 32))
 (segment (start 90.932 71.628) (end 104.648 71.628) (width 0.2) (layer "F.Cu") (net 32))
 (segment (start 83.058 67.056) (end 86.36 67.056) (width 0.2) (layer "F.Cu") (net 32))
 (via (at 86.36 67.056) (size 0.6) (drill 0.3) (layers "F.Cu" "B.Cu") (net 32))
 (segment (start 86.346 65.612) (end 86.346 67.042) (width 0.2) (layer "B.Cu") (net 32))
 (segment (start 86.346 67.042) (end 86.36 67.056) (width 0.2) (layer "B.Cu") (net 32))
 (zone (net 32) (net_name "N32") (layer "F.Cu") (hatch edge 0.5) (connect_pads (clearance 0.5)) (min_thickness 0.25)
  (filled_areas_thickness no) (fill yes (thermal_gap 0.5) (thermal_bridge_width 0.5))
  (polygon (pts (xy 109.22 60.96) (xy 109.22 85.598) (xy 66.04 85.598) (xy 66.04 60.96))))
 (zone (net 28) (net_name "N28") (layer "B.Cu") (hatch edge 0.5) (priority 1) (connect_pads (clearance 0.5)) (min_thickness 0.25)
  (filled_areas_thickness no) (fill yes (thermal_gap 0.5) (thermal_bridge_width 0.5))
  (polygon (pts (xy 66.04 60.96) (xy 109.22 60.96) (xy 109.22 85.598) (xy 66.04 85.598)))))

